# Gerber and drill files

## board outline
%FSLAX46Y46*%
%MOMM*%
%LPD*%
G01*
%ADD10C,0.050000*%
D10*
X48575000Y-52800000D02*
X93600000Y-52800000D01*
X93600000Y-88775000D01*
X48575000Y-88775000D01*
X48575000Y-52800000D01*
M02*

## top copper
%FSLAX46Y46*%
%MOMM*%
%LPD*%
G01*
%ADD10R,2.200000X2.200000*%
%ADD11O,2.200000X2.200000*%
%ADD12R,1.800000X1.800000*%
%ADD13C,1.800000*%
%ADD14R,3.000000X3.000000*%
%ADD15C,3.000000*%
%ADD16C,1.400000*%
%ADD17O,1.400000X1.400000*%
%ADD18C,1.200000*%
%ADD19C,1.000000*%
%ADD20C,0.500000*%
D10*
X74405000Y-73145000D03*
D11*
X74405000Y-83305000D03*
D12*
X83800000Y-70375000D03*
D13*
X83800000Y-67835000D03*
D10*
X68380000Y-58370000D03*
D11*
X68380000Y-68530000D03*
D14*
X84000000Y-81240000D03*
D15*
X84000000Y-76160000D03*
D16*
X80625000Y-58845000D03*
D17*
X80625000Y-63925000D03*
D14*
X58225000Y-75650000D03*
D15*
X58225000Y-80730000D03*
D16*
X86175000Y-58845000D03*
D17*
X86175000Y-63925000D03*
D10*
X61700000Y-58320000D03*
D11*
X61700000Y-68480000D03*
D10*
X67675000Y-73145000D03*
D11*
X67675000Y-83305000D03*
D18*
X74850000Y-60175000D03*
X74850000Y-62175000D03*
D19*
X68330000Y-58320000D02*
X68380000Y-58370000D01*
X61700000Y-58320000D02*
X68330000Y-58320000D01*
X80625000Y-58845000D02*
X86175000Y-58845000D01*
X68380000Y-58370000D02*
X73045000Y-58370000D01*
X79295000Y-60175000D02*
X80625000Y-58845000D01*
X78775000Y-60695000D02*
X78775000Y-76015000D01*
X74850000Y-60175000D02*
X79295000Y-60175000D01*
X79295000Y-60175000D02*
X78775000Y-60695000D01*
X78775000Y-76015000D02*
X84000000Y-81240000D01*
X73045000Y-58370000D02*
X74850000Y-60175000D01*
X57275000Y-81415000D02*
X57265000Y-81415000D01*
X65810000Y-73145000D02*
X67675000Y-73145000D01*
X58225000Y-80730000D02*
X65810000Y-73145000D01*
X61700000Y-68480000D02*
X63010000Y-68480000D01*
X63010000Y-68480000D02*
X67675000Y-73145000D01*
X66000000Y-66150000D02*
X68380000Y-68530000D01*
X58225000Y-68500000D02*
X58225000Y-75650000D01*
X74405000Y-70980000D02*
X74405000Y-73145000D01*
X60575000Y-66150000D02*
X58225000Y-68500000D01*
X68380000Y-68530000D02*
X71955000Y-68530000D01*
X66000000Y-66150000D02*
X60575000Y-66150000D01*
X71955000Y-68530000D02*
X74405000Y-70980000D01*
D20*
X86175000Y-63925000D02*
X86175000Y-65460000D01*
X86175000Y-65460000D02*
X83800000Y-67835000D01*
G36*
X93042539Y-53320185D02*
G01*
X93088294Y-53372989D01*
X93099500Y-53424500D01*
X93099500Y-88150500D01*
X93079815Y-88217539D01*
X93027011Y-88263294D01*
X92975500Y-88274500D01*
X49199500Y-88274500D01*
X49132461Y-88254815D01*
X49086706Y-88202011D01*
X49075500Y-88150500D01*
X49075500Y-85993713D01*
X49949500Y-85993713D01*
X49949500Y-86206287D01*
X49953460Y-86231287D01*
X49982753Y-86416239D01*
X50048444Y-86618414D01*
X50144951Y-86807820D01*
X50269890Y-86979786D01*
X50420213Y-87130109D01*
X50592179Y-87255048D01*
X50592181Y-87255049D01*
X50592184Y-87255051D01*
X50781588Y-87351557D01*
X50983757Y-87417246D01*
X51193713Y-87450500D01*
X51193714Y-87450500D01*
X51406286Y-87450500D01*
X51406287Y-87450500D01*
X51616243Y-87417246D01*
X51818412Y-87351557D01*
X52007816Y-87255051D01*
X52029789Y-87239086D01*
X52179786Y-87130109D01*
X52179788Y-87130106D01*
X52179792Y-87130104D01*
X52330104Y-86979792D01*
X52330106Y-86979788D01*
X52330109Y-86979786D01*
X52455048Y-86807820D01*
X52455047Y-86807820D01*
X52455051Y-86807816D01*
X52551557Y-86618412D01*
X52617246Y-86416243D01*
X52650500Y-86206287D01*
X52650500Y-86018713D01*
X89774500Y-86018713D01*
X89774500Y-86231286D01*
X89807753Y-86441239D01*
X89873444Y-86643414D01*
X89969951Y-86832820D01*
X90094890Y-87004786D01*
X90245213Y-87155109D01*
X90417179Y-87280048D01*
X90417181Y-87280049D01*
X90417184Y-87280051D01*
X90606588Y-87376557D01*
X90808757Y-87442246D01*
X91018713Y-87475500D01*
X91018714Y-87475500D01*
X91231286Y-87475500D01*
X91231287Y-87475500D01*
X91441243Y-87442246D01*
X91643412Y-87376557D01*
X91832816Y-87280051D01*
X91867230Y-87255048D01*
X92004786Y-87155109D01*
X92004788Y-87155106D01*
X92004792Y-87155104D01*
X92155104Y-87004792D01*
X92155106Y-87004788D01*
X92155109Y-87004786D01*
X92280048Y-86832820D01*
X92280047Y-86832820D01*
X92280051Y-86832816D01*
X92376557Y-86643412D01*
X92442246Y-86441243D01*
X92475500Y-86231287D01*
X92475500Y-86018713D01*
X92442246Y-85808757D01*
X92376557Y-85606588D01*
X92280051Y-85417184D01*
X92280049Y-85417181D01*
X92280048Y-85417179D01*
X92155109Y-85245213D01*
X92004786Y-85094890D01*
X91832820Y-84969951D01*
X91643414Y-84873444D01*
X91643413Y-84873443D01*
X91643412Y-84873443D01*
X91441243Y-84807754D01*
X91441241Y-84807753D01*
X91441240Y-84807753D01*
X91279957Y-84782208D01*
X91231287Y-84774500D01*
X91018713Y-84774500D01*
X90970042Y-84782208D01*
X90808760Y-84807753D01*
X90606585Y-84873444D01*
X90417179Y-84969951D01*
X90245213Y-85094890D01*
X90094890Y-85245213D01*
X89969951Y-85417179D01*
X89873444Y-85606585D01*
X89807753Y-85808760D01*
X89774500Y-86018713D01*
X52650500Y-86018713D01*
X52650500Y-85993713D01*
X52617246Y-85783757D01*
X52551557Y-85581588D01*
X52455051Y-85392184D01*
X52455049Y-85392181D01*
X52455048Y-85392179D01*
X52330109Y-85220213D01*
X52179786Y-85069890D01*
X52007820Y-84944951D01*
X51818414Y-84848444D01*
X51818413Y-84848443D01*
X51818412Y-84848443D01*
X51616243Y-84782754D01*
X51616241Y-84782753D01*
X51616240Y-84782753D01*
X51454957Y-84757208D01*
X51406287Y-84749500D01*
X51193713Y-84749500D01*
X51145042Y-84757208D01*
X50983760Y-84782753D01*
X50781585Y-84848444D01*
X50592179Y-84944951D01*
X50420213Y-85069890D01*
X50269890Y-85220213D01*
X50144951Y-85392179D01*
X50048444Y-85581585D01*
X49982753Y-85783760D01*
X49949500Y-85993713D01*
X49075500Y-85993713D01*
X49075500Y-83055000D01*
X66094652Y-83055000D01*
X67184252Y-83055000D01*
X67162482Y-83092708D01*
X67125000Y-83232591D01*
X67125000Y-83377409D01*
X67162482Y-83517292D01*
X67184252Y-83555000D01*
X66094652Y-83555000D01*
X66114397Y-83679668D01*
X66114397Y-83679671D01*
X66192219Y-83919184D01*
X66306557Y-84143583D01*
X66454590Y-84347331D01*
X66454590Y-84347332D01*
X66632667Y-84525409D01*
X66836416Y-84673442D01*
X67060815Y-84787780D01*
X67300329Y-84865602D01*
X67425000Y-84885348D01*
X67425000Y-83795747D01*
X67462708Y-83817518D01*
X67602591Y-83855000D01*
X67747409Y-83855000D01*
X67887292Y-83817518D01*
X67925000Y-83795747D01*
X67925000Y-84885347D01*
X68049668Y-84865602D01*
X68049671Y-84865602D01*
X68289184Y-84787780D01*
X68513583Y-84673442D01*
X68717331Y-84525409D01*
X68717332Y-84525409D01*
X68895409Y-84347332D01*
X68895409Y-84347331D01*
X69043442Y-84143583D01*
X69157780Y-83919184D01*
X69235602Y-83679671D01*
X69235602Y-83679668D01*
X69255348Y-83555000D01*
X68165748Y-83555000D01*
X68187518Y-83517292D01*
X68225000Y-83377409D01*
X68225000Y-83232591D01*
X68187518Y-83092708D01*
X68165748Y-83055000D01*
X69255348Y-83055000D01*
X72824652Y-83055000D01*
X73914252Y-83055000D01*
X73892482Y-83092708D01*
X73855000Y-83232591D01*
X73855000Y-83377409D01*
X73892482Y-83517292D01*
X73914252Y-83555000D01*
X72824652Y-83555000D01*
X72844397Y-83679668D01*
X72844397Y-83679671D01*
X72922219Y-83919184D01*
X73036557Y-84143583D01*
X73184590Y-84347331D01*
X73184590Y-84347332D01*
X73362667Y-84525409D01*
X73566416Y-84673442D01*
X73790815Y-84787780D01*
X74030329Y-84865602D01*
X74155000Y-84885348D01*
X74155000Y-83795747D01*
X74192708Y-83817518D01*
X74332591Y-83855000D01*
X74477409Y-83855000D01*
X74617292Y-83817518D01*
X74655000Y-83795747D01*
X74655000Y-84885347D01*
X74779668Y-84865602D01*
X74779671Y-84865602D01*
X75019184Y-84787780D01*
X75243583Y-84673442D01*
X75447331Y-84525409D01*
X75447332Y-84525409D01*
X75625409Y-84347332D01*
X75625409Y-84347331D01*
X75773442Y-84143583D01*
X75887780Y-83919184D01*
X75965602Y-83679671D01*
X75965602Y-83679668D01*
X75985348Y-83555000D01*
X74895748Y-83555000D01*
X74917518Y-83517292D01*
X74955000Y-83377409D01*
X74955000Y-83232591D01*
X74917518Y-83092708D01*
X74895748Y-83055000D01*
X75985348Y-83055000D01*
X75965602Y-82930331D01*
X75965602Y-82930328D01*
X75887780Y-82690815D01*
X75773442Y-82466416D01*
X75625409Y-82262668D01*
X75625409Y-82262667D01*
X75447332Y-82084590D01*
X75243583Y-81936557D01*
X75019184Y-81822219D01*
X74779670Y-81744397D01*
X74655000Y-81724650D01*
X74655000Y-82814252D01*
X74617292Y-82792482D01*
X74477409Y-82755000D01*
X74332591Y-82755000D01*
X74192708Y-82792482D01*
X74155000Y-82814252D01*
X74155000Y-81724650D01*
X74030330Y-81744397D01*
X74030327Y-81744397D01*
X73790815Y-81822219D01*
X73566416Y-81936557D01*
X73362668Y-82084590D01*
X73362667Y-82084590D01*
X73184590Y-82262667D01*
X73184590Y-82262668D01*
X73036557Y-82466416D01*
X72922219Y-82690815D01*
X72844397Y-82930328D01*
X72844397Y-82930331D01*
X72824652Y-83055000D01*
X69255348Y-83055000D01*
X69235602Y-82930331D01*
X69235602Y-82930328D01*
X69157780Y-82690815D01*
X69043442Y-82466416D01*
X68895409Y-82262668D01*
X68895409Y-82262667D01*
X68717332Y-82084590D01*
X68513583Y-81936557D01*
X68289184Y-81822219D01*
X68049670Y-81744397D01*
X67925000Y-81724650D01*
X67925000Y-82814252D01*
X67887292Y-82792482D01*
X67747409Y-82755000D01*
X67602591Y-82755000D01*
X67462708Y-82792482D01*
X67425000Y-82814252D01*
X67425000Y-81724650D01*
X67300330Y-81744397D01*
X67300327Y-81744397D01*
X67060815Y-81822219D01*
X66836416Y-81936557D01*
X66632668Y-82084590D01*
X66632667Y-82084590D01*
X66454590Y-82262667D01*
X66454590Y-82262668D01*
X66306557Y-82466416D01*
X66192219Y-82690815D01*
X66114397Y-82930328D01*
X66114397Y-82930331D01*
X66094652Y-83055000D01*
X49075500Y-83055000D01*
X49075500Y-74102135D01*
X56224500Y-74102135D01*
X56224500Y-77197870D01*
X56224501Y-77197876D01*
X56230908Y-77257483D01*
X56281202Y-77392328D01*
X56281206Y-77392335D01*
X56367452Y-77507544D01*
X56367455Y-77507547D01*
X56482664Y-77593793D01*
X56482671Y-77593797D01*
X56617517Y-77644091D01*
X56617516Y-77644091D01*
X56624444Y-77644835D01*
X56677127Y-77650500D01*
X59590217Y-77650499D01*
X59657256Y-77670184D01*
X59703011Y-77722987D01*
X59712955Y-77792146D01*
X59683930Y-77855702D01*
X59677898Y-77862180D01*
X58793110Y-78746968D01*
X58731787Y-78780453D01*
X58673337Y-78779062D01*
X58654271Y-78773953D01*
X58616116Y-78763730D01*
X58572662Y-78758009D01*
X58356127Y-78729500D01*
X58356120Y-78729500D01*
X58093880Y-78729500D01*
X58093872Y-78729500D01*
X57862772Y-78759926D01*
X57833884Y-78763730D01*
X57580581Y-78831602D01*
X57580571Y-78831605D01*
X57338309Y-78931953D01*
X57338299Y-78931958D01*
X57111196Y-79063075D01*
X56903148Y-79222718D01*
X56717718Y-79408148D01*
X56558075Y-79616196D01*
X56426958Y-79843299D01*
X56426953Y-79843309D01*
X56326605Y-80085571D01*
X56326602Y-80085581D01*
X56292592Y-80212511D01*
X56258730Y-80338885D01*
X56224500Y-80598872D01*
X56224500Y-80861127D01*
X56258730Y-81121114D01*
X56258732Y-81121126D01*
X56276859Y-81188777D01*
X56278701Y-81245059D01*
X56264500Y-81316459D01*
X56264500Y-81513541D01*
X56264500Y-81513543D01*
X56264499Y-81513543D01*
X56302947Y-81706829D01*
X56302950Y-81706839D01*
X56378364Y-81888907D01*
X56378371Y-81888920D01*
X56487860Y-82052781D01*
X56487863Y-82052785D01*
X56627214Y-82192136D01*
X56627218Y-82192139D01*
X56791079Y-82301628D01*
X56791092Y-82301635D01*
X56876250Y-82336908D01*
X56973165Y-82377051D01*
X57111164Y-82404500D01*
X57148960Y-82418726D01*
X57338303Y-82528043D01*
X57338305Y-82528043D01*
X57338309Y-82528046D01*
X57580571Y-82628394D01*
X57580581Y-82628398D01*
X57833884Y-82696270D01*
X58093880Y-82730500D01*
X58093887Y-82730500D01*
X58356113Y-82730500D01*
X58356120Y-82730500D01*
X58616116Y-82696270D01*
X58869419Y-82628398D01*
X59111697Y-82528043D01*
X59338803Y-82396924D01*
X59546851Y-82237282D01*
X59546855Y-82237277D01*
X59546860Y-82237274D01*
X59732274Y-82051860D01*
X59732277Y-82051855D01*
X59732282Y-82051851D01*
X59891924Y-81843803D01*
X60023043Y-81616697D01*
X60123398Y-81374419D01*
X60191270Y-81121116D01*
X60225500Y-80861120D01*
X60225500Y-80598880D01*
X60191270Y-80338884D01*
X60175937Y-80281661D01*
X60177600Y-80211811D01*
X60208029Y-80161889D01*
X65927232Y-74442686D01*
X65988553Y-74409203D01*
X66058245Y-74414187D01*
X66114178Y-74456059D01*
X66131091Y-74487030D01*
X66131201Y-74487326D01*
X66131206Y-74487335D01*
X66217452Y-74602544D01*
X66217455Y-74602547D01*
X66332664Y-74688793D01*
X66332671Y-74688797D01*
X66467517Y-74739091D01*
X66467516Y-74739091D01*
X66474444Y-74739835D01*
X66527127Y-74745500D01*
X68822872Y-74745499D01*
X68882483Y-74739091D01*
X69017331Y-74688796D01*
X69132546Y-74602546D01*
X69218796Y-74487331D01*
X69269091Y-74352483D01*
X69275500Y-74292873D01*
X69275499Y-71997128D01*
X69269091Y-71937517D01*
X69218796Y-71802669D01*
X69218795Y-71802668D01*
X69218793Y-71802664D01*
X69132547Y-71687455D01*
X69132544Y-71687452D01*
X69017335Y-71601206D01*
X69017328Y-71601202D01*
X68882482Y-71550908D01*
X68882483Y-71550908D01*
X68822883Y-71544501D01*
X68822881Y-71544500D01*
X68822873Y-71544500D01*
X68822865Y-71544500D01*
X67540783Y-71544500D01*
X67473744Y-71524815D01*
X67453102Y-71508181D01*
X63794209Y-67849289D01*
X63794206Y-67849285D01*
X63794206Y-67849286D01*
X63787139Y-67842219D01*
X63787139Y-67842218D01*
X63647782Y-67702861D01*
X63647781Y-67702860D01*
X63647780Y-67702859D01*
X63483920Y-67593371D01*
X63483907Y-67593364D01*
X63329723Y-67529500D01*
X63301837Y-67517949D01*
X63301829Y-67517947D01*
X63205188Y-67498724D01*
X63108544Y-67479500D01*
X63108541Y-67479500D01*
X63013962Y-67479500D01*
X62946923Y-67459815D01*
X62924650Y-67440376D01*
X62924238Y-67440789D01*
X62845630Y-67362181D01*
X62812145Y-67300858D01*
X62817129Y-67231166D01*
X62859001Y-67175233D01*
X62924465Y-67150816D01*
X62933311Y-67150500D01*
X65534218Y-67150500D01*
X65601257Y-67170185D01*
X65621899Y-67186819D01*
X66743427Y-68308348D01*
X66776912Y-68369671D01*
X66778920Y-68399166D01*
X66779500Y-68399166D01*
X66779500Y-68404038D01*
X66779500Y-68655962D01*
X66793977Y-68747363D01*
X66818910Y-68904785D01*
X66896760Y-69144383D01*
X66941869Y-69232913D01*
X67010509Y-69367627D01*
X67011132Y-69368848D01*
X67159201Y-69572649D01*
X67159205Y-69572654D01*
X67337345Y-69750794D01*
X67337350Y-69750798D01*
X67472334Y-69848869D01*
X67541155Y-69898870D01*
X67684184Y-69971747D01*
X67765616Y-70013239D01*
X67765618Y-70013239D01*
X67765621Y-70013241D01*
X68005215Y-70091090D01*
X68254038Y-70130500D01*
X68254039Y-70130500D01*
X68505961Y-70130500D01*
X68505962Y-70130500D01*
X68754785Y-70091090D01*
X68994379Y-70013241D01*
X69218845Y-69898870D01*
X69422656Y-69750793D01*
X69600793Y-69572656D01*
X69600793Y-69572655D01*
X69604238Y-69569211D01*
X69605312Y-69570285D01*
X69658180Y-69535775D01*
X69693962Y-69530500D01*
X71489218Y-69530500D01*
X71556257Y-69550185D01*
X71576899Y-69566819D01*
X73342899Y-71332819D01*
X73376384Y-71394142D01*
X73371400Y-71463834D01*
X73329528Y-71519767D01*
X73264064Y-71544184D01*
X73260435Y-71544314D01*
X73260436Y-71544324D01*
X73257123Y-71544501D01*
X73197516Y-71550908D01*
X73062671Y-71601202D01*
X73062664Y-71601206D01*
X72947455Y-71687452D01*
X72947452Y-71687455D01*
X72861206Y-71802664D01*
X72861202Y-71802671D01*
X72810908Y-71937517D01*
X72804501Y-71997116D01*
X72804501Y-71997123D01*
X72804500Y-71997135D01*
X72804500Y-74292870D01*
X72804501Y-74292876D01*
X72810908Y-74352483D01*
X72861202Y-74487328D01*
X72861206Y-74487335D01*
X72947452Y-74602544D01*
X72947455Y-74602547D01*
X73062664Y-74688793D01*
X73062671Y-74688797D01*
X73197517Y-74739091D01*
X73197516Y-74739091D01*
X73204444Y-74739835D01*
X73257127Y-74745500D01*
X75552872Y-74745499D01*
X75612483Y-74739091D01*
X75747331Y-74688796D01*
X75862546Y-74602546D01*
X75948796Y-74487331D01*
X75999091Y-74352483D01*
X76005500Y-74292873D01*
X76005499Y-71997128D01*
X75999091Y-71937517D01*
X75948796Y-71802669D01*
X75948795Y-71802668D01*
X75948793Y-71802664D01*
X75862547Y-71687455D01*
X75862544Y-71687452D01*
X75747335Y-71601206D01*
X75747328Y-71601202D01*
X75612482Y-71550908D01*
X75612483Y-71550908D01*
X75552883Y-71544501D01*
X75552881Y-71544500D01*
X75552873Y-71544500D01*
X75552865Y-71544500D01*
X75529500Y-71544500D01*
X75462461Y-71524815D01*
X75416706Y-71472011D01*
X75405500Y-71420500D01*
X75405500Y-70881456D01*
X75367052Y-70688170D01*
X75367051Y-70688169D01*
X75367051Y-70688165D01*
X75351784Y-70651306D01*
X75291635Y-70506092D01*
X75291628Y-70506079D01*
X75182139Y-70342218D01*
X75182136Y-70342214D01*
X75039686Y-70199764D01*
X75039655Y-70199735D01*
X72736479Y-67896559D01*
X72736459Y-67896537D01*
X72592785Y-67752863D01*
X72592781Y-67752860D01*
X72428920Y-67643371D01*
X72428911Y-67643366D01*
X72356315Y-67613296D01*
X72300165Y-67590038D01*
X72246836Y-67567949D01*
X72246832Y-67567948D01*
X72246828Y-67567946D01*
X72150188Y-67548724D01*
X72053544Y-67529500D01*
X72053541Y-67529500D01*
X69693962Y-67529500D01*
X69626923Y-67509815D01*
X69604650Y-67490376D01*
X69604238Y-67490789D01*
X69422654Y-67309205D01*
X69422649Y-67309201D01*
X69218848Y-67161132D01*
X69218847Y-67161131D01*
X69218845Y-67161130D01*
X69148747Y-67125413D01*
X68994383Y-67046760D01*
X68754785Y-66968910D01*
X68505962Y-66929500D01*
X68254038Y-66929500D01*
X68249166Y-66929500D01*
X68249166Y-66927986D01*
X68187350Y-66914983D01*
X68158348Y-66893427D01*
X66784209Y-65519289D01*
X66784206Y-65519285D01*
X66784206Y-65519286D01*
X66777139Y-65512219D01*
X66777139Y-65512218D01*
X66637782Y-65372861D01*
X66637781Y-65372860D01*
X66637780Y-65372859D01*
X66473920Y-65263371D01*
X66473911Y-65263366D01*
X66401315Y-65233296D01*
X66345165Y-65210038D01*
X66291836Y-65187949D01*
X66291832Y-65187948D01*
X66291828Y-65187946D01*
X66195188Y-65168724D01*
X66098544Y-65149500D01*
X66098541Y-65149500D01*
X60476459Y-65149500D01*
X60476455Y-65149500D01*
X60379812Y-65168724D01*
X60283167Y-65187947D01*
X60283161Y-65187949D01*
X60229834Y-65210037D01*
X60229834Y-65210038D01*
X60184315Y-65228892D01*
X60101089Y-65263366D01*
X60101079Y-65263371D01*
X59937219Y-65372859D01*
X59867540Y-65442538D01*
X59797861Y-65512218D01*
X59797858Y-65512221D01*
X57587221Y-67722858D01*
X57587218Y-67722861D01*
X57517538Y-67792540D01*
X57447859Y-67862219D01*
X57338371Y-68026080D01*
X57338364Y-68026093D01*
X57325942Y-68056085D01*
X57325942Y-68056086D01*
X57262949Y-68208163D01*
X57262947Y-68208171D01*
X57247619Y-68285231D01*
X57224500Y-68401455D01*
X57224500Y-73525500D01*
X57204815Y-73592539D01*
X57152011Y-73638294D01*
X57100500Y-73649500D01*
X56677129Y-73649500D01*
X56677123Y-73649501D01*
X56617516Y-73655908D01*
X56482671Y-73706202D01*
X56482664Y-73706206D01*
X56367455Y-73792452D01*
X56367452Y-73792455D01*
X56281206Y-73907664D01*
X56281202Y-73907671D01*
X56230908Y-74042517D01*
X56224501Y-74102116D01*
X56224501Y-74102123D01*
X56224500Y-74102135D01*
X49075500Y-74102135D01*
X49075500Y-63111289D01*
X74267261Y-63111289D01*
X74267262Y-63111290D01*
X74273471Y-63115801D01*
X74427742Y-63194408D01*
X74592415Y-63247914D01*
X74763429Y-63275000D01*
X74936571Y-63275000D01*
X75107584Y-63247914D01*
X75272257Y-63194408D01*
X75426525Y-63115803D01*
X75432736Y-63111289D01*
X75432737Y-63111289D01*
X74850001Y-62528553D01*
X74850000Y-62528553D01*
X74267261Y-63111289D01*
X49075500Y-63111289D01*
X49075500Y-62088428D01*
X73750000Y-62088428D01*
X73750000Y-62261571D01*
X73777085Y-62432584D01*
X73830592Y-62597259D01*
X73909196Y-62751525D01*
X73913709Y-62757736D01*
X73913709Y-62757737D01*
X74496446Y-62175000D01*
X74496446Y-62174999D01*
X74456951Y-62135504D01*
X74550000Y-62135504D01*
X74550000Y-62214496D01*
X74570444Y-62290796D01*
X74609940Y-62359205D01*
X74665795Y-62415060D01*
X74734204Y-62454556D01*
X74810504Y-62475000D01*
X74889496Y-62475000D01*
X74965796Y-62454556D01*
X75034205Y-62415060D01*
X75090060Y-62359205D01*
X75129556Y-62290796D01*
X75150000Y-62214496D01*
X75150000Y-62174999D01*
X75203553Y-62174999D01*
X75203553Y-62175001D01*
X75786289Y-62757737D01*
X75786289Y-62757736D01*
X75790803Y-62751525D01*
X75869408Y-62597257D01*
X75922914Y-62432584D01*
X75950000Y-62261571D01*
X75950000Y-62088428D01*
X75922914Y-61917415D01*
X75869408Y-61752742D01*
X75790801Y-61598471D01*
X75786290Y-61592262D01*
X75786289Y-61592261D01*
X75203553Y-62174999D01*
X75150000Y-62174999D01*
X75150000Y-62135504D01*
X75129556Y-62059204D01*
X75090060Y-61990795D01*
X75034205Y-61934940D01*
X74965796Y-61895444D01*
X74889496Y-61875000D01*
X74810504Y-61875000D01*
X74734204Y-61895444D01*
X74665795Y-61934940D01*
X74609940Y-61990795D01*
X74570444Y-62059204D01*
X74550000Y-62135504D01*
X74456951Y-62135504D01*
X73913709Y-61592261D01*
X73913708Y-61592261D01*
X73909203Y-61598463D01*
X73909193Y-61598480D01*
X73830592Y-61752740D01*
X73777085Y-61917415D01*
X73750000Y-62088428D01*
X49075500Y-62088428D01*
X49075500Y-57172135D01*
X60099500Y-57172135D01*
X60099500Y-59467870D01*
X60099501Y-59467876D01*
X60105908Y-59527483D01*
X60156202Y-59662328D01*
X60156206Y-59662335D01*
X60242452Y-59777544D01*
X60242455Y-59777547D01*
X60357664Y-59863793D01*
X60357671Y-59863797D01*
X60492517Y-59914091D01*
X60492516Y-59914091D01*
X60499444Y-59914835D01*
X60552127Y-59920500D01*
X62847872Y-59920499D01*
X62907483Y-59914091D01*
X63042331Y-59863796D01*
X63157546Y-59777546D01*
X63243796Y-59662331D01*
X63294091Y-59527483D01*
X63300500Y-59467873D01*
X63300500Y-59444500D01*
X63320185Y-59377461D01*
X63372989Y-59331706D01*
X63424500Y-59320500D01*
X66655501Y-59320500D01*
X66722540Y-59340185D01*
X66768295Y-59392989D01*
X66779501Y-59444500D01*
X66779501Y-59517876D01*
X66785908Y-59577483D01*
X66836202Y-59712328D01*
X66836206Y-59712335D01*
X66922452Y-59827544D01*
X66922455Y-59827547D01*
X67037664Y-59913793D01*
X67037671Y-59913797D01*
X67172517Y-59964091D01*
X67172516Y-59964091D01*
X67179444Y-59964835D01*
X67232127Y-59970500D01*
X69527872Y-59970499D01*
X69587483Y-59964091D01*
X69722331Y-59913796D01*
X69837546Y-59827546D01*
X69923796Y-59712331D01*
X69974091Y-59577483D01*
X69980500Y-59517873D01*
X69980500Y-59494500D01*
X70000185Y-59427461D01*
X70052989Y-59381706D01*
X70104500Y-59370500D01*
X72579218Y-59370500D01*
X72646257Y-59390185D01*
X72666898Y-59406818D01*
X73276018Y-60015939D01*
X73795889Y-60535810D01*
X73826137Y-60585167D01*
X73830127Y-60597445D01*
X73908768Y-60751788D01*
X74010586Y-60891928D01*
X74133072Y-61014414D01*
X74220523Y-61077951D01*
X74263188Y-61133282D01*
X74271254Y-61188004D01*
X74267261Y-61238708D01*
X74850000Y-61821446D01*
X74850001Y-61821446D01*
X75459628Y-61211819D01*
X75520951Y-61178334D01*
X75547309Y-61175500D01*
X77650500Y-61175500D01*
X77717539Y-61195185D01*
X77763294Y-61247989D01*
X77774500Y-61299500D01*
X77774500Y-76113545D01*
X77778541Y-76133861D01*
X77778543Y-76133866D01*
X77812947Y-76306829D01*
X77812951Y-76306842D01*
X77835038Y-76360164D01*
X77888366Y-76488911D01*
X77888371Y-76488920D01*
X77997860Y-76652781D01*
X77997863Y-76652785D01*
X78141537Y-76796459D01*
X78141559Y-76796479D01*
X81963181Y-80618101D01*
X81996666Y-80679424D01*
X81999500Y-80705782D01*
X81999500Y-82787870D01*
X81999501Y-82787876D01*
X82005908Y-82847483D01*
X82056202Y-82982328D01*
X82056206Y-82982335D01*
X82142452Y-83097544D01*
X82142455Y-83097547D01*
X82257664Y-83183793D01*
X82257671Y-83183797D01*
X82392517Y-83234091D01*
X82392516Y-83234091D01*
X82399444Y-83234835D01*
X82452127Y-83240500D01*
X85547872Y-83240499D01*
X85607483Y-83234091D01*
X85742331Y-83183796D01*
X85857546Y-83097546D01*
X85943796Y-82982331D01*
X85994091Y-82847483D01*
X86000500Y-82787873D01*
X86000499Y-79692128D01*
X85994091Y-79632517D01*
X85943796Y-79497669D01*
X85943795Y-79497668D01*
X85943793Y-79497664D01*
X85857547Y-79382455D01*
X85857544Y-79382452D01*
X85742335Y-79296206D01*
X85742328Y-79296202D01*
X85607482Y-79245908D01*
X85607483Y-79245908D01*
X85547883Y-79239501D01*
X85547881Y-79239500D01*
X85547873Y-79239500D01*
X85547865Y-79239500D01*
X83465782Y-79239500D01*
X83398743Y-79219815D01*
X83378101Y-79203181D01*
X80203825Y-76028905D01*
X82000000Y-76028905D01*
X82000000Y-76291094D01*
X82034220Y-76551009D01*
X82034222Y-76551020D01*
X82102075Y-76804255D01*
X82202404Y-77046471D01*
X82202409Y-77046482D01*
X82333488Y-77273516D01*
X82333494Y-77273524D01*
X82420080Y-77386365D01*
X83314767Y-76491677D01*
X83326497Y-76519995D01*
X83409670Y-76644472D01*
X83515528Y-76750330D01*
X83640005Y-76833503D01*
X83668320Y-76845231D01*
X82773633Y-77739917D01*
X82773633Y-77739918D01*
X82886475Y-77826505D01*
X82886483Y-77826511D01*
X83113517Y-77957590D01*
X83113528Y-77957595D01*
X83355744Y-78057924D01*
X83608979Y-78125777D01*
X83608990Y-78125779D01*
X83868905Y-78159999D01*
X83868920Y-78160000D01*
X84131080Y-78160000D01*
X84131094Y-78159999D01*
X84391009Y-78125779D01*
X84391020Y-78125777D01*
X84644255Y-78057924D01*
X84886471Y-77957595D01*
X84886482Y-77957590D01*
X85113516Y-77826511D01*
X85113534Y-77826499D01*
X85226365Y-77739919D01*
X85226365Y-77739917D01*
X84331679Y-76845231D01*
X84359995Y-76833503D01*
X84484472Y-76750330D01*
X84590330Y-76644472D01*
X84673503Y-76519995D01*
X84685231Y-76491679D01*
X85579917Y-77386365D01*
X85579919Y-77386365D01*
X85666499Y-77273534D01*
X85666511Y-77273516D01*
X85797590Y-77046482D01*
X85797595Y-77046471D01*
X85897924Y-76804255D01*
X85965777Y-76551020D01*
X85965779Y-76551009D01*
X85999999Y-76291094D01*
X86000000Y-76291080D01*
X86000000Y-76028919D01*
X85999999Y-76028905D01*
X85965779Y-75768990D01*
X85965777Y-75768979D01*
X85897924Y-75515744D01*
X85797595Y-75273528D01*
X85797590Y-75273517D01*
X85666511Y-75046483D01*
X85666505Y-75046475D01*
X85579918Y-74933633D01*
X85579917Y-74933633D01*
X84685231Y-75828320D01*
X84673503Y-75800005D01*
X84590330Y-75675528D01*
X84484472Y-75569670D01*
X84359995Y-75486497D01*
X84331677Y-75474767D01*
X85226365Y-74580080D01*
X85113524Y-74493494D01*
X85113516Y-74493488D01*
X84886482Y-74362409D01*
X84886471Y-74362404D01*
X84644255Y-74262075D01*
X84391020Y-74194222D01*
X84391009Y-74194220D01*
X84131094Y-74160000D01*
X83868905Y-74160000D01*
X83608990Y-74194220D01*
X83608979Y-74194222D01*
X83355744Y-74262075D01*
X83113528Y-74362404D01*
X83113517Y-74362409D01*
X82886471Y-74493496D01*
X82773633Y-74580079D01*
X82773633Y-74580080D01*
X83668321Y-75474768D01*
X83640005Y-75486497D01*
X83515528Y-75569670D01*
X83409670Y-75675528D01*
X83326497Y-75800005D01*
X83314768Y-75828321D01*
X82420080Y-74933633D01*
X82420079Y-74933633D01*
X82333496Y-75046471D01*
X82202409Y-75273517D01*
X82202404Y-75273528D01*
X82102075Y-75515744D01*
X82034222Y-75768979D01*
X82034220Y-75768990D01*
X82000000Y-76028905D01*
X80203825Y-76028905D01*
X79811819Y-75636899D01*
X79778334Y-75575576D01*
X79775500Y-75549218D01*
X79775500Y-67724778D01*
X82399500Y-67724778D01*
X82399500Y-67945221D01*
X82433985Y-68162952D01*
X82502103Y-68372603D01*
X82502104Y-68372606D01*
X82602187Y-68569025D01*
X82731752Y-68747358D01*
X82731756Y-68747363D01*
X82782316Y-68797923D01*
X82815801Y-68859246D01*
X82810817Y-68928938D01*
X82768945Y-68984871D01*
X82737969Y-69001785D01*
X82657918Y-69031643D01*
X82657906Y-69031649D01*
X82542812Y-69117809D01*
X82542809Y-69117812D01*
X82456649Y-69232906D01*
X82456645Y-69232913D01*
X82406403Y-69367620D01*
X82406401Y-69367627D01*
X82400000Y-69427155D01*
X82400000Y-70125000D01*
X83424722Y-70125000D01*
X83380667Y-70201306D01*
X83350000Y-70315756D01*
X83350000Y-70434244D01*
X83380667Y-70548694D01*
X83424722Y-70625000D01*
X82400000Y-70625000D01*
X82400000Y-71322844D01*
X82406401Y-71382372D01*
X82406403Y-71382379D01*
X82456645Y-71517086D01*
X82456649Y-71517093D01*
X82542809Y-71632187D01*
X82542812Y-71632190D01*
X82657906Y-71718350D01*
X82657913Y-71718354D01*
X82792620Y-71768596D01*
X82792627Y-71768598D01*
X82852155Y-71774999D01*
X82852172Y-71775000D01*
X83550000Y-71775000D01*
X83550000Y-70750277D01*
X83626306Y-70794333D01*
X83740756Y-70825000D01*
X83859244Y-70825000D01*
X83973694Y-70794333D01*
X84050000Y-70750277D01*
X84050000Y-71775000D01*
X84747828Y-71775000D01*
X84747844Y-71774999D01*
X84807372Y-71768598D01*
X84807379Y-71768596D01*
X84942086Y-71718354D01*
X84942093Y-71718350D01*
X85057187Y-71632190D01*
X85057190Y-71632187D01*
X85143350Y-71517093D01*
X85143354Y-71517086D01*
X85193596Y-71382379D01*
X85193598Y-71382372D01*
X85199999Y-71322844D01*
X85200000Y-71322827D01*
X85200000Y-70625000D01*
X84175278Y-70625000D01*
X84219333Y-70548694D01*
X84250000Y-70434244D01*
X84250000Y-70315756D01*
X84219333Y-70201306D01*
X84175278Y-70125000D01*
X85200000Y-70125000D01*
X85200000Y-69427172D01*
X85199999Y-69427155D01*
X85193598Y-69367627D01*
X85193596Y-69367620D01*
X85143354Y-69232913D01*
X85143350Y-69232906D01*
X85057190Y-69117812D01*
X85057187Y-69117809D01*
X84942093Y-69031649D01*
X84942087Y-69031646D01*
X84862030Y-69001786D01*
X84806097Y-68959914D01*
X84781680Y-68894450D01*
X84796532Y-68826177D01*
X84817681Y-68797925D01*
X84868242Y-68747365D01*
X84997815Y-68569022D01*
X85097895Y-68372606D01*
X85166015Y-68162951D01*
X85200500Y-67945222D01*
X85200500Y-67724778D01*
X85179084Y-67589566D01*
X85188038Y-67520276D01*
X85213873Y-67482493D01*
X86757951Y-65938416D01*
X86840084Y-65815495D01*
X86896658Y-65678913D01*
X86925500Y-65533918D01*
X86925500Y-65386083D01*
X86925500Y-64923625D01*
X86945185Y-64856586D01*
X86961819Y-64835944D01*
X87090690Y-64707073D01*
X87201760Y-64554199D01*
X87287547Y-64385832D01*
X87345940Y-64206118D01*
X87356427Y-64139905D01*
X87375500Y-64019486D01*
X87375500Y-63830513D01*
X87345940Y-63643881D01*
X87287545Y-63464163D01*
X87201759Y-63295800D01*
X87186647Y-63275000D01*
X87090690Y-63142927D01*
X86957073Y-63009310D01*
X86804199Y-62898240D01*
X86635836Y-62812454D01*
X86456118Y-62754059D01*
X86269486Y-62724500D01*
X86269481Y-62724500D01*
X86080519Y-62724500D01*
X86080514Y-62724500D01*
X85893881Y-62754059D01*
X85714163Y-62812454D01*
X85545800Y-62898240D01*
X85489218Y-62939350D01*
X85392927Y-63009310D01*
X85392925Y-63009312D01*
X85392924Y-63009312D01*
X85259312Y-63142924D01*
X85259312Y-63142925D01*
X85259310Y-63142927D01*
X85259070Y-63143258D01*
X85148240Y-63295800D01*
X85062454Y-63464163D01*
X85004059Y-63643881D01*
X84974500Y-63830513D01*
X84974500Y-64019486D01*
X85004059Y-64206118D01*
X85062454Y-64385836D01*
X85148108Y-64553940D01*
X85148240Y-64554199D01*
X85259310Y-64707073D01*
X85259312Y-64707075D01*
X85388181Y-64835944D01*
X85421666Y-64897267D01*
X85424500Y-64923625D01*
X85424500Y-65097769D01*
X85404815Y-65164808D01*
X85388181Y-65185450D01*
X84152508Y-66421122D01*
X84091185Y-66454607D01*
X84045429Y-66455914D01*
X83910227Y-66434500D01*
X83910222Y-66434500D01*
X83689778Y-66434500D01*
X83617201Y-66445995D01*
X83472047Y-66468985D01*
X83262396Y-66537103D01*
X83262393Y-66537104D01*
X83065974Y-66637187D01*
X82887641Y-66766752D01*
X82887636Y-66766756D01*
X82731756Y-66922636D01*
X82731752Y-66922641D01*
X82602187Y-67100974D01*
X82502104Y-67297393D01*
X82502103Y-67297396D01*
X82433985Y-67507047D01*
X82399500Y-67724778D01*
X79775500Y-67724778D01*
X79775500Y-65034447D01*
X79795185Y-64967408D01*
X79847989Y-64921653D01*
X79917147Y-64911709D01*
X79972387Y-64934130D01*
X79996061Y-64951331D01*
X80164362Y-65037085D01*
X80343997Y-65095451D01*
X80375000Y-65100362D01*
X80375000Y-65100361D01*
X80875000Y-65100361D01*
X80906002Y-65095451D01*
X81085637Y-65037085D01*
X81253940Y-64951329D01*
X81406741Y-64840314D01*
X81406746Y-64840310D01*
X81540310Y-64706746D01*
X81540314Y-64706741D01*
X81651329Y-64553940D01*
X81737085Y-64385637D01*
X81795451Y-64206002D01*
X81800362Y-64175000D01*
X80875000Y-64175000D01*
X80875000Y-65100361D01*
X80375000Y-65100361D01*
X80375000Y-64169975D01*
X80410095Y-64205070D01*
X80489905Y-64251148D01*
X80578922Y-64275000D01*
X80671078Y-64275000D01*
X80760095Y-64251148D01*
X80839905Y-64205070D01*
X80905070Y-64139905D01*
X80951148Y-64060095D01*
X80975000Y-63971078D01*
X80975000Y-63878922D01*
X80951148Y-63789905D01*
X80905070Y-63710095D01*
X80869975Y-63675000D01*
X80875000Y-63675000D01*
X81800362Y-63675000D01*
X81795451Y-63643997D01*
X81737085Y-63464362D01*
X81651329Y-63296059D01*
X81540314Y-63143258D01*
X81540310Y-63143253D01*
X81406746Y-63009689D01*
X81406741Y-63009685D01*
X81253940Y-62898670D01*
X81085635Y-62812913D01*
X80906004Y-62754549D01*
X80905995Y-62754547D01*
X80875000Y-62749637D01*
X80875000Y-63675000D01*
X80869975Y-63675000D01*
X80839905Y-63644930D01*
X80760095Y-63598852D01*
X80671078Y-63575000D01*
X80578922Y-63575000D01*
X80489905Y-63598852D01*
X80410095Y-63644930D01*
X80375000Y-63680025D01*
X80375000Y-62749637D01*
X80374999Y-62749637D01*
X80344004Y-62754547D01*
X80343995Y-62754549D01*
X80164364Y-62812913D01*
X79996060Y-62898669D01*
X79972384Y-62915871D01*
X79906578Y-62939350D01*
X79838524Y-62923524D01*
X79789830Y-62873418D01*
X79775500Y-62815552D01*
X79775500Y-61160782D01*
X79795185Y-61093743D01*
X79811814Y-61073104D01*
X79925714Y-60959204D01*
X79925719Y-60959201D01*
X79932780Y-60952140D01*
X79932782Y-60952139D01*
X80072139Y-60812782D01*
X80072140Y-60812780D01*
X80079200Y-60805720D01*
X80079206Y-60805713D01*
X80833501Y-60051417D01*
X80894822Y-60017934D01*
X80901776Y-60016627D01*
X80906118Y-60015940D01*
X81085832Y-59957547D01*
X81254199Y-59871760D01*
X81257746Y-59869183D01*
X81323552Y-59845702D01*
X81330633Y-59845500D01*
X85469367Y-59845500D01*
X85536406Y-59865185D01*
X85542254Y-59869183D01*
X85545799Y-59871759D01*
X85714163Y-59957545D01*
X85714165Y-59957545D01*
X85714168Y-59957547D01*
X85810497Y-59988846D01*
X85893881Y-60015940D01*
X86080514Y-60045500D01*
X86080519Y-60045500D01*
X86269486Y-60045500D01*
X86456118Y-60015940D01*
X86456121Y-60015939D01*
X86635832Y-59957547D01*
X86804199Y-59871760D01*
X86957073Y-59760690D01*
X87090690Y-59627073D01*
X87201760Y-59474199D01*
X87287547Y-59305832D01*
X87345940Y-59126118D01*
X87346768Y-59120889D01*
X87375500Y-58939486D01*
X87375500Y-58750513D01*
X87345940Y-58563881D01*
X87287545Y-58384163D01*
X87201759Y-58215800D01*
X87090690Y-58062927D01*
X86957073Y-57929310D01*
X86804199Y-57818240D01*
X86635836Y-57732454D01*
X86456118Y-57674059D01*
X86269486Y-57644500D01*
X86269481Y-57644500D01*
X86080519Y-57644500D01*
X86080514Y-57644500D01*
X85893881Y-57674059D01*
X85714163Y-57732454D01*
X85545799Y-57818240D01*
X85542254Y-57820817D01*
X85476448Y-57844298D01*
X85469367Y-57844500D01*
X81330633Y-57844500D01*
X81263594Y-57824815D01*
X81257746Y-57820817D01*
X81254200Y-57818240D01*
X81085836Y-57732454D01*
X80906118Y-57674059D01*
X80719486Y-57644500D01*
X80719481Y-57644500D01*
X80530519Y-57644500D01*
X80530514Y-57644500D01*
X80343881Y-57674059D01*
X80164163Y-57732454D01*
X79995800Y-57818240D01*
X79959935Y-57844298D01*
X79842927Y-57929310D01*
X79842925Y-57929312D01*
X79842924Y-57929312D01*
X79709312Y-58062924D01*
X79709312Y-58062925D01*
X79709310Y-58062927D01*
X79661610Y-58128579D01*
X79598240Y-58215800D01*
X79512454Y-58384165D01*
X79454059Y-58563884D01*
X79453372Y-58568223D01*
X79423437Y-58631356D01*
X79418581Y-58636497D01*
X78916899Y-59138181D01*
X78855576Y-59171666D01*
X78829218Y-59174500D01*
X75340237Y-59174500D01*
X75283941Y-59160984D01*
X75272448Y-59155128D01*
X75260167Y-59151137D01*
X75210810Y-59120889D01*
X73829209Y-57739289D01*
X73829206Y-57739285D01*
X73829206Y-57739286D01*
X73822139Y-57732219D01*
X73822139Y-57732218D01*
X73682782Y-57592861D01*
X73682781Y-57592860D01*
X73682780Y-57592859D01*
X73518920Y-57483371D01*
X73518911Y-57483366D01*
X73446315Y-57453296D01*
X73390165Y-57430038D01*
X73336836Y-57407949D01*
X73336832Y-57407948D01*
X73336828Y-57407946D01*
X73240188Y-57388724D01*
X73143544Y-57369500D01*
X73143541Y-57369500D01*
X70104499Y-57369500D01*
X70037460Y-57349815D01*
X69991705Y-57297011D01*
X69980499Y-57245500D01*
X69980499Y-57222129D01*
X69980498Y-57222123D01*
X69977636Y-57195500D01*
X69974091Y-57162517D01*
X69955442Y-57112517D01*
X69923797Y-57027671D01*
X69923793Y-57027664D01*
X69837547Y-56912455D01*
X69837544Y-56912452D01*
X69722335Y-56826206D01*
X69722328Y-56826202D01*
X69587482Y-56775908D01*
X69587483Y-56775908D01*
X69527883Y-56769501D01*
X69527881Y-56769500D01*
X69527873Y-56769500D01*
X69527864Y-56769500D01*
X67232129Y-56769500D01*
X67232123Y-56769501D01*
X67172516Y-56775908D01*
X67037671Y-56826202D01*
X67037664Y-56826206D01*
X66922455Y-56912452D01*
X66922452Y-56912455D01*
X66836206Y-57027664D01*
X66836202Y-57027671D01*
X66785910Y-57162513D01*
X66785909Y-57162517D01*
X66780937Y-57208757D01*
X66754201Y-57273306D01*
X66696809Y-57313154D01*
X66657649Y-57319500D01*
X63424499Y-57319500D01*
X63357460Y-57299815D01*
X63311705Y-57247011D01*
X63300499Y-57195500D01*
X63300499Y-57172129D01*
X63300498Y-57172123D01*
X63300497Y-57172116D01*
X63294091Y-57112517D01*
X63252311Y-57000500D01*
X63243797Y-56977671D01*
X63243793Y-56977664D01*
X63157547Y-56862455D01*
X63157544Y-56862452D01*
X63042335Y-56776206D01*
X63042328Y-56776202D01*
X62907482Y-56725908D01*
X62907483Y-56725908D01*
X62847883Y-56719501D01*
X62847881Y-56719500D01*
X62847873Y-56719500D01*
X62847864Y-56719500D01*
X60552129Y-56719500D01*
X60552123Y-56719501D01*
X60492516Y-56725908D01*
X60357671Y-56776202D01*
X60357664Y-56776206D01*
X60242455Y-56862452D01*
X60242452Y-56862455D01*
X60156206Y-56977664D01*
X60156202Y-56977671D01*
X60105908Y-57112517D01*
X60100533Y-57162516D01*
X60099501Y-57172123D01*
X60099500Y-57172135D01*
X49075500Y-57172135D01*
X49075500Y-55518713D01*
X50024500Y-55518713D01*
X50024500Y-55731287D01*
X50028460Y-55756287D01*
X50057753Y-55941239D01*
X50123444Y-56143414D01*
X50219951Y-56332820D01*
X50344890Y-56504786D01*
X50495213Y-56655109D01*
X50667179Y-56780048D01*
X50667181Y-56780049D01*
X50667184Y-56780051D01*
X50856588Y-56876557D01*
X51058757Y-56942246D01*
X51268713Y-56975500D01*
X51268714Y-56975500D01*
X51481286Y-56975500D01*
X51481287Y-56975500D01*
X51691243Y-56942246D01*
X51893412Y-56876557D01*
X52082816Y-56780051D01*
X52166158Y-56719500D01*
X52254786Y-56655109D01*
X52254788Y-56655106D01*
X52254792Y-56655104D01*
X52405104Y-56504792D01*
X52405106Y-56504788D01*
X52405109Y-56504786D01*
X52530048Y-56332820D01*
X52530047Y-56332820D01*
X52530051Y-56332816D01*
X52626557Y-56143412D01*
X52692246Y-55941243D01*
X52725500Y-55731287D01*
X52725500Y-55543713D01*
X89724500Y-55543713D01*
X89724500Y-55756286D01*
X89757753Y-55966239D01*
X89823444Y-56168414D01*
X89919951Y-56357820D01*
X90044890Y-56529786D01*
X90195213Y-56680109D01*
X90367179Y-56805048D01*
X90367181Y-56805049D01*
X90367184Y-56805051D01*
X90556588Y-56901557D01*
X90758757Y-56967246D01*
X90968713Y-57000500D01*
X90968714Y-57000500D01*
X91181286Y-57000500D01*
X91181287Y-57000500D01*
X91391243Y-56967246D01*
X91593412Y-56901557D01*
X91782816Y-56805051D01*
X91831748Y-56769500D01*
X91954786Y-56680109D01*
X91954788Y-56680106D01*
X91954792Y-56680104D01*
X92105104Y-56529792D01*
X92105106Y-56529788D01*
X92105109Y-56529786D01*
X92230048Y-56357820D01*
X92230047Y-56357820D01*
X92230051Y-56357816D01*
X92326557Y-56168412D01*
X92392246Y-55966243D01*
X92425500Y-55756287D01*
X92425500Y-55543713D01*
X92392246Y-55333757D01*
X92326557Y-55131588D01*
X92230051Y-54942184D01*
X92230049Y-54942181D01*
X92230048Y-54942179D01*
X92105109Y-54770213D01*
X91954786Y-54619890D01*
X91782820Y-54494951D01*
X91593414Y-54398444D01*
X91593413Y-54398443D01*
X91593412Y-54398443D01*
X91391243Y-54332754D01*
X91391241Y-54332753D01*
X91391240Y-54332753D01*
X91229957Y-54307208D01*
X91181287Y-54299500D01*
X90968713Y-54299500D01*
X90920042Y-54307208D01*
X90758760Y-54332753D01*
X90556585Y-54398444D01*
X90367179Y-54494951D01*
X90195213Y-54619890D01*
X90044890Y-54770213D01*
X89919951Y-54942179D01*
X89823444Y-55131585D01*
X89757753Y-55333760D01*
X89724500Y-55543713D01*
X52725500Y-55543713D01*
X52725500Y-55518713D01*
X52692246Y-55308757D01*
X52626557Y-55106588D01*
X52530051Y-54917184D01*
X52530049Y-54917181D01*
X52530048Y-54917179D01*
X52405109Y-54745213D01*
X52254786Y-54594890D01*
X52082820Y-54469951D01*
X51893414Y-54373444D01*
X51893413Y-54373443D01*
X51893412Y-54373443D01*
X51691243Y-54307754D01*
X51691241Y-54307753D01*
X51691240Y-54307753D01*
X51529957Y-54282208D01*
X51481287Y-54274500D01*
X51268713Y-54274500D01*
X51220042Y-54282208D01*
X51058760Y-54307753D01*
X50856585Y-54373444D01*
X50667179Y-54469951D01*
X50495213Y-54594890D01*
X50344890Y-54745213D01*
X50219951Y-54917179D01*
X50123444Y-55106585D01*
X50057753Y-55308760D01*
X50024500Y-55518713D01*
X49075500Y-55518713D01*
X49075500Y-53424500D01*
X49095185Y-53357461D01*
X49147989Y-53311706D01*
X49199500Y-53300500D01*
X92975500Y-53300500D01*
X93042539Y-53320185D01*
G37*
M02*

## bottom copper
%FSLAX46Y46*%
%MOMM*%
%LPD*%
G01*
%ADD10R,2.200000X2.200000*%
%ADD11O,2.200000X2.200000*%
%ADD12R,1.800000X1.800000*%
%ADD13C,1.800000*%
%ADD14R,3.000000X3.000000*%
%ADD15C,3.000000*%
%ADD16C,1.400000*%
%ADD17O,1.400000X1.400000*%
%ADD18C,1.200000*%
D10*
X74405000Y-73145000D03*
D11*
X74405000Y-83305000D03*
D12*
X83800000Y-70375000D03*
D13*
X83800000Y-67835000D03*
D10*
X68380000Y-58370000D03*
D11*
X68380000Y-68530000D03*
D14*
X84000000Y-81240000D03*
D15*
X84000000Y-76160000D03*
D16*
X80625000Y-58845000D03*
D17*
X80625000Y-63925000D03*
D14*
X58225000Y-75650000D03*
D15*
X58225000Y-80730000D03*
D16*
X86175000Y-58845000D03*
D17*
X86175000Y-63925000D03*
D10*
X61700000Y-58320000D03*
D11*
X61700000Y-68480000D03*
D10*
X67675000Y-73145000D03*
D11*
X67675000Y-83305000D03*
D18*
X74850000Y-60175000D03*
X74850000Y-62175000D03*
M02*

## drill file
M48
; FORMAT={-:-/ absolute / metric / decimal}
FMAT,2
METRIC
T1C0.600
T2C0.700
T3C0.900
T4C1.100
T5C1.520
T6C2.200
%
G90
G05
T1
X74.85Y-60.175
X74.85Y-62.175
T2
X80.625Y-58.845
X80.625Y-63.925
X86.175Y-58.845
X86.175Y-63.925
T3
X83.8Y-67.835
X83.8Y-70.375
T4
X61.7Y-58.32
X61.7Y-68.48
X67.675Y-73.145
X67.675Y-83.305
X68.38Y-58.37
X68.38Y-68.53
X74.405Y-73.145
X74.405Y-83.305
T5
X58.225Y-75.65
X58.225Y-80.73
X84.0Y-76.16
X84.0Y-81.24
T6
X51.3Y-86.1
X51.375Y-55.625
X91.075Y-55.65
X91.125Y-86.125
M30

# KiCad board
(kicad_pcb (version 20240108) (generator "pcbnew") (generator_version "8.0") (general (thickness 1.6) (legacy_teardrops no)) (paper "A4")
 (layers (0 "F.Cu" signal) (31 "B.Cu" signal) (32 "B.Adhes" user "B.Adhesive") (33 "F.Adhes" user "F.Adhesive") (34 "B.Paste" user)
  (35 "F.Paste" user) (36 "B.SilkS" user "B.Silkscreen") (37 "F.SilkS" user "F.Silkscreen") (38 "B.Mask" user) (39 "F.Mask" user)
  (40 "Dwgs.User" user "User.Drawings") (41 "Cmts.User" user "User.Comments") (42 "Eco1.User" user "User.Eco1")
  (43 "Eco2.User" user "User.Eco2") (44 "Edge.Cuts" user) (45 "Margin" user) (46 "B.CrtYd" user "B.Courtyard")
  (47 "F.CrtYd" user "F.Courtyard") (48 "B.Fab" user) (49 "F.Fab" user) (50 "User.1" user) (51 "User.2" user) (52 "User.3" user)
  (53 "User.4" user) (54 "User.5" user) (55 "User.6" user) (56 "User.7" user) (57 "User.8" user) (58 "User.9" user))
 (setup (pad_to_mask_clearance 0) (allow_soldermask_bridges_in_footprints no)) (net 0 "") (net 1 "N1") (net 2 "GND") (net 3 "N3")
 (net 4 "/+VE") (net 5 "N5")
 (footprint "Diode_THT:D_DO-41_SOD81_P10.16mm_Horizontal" (layer "F.Cu") (at 74.405 73.145 -90)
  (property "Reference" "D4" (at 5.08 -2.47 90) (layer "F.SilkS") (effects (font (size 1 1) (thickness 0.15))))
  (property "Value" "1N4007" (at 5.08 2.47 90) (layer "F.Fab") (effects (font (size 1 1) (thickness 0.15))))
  (pad "1" thru_hole rect (at 0 0 270) (size 2.2 2.2) (drill 1.1) (layers "*.Cu" "*.Mask") (remove_unused_layers no) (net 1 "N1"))
  (pad "2" thru_hole oval (at 10.16 0 270) (size 2.2 2.2) (drill 1.1) (layers "*.Cu" "*.Mask") (remove_unused_layers no) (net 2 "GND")))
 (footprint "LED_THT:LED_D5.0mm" (layer "F.Cu") (at 83.8 70.375 90)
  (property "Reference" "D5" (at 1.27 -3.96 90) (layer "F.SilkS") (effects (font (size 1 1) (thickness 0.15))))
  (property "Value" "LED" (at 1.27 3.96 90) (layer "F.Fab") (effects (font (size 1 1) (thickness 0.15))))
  (pad "1" thru_hole rect (at 0 0 90) (size 1.8 1.8) (drill 0.9) (layers "*.Cu" "*.Mask") (remove_unused_layers no) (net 2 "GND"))
  (pad "2" thru_hole circle (at 2.54 0 90) (size 1.8 1.8) (drill 0.9) (layers "*.Cu" "*.Mask") (remove_unused_layers no) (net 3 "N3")))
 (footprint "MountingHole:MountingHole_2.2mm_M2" (layer "F.Cu") (at 51.375 55.625)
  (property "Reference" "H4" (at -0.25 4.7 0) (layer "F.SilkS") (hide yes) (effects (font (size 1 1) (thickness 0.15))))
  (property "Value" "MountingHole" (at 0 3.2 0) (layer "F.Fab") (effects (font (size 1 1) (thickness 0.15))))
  (pad "" np_thru_hole circle (at 0 0) (size 2.2 2.2) (drill 2.2) (layers "*.Cu" "*.Mask")))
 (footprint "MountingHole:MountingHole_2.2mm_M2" (layer "F.Cu") (at 91.125 86.125)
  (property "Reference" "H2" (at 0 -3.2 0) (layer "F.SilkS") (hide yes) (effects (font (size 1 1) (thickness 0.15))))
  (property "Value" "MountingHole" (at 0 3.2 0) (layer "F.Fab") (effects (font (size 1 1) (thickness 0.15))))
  (pad "" np_thru_hole circle (at 0 0) (size 2.2 2.2) (drill 2.2) (layers "*.Cu" "*.Mask")))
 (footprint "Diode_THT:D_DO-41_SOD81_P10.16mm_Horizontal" (layer "F.Cu") (at 68.38 58.37 -90)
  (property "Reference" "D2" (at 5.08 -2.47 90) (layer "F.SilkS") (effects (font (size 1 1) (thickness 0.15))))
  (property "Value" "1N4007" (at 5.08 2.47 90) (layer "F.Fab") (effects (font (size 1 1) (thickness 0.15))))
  (pad "1" thru_hole rect (at 0 0 270) (size 2.2 2.2) (drill 1.1) (layers "*.Cu" "*.Mask") (remove_unused_layers no) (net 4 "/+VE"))
  (pad "2" thru_hole oval (at 10.16 0 270) (size 2.2 2.2) (drill 1.1) (layers "*.Cu" "*.Mask") (remove_unused_layers no) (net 1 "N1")))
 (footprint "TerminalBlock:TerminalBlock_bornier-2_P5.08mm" (layer "F.Cu") (at 84 81.24 90)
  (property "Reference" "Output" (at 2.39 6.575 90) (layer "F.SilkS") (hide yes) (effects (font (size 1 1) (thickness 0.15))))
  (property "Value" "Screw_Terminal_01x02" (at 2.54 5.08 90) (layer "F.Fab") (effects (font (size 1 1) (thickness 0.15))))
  (pad "1" thru_hole rect (at 0 0 90) (size 3 3) (drill 1.52) (layers "*.Cu" "*.Mask") (remove_unused_layers no) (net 4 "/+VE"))
  (pad "2" thru_hole circle (at 5.08 0 90) (size 3 3) (drill 1.52) (layers "*.Cu" "*.Mask") (remove_unused_layers no) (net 2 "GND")))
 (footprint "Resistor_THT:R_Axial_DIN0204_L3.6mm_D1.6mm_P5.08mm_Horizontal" (layer "F.Cu") (at 80.625 58.845 -90)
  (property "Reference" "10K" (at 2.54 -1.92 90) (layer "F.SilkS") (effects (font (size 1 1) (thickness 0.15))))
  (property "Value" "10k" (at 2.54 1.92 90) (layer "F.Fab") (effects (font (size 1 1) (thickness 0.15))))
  (pad "1" thru_hole circle (at 0 0 270) (size 1.4 1.4) (drill 0.7) (layers "*.Cu" "*.Mask") (remove_unused_layers no) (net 4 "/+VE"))
  (pad "2" thru_hole oval (at 5.08 0 270) (size 1.4 1.4) (drill 0.7) (layers "*.Cu" "*.Mask") (remove_unused_layers no) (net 2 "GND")))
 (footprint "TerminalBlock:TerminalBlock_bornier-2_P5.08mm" (layer "F.Cu") (at 58.225 75.65 -90)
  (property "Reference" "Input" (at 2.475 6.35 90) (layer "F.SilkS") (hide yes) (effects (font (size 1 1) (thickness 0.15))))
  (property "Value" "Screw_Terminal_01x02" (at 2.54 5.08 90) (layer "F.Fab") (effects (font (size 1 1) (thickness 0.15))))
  (pad "1" thru_hole rect (at 0 0 270) (size 3 3) (drill 1.52) (layers "*.Cu" "*.Mask") (remove_unused_layers no) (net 1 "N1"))
  (pad "2" thru_hole circle (at 5.08 0 270) (size 3 3) (drill 1.52) (layers "*.Cu" "*.Mask") (remove_unused_layers no) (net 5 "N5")))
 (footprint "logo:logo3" (layer "F.Cu") (at 54.3 62.625)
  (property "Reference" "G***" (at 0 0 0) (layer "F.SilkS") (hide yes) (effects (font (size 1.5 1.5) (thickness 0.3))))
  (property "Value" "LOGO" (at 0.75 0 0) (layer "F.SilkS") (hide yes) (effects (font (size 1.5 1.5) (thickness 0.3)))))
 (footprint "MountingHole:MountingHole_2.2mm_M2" (layer "F.Cu") (at 51.3 86.1)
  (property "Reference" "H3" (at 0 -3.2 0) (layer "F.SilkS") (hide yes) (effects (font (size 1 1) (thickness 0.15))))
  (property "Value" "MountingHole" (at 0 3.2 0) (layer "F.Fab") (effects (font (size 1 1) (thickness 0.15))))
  (pad "" np_thru_hole circle (at 0 0) (size 2.2 2.2) (drill 2.2) (layers "*.Cu" "*.Mask")))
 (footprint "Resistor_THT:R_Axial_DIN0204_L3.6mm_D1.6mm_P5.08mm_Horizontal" (layer "F.Cu") (at 86.175 58.845 -90)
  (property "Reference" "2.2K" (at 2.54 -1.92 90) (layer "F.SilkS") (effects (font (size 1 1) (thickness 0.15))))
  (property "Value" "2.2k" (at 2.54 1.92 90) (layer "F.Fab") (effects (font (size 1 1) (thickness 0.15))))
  (pad "1" thru_hole circle (at 0 0 270) (size 1.4 1.4) (drill 0.7) (layers "*.Cu" "*.Mask") (remove_unused_layers no) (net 4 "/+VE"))
  (pad "2" thru_hole oval (at 5.08 0 270) (size 1.4 1.4) (drill 0.7) (layers "*.Cu" "*.Mask") (remove_unused_layers no) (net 3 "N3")))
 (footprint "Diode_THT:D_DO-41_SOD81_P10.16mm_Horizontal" (layer "F.Cu") (at 61.7 58.32 -90)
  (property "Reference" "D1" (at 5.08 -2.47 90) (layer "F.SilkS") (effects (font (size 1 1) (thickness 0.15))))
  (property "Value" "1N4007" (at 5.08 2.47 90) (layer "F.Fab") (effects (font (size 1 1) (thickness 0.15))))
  (pad "1" thru_hole rect (at 0 0 270) (size 2.2 2.2) (drill 1.1) (layers "*.Cu" "*.Mask") (remove_unused_layers no) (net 4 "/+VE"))
  (pad "2" thru_hole oval (at 10.16 0 270) (size 2.2 2.2) (drill 1.1) (layers "*.Cu" "*.Mask") (remove_unused_layers no) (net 5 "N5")))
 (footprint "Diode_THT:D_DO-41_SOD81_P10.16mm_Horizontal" (layer "F.Cu") (at 67.675 73.145 -90)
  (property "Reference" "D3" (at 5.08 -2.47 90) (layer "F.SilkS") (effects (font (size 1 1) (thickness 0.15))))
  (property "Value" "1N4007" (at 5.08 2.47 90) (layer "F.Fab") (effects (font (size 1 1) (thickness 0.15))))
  (pad "1" thru_hole rect (at 0 0 270) (size 2.2 2.2) (drill 1.1) (layers "*.Cu" "*.Mask") (remove_unused_layers no) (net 5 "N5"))
  (pad "2" thru_hole oval (at 10.16 0 270) (size 2.2 2.2) (drill 1.1) (layers "*.Cu" "*.Mask") (remove_unused_layers no) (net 2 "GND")))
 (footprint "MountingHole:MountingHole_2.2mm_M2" (layer "F.Cu") (at 91.075 55.65)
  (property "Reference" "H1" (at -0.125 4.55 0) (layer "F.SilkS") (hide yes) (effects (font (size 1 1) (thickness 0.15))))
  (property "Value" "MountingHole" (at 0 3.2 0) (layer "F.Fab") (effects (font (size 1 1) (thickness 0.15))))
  (pad "" np_thru_hole circle (at 0 0) (size 2.2 2.2) (drill 2.2) (layers "*.Cu" "*.Mask")))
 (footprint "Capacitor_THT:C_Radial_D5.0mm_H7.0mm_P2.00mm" (layer "F.Cu") (at 74.85 60.175 -90)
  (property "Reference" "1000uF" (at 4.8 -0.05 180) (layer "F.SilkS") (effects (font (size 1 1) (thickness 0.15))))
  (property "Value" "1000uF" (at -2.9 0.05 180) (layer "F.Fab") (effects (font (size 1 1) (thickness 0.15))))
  (pad "1" thru_hole circle (at 0 0 270) (size 1.2 1.2) (drill 0.6) (layers "*.Cu" "*.Mask") (remove_unused_layers no) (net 4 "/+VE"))
  (pad "2" thru_hole circle (at 2 0 270) (size 1.2 1.2) (drill 0.6) (layers "*.Cu" "*.Mask") (remove_unused_layers no) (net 2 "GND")))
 (gr_rect (start 48.575 52.8) (end 93.6 88.775) (stroke (width 0.05) (type default)) (fill none) (layer "Edge.Cuts"))
 (segment (start 68.33 58.32) (end 68.38 58.37) (width 1) (layer "F.Cu") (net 4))
 (segment (start 61.7 58.32) (end 68.33 58.32) (width 1) (layer "F.Cu") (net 4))
 (segment (start 80.625 58.845) (end 86.175 58.845) (width 1) (layer "F.Cu") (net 4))
 (segment (start 68.38 58.37) (end 73.045 58.37) (width 1) (layer "F.Cu") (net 4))
 (segment (start 79.295 60.175) (end 80.625 58.845) (width 1) (layer "F.Cu") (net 4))
 (segment (start 78.775 60.695) (end 78.775 76.015) (width 1) (layer "F.Cu") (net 4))
 (segment (start 74.85 60.175) (end 79.295 60.175) (width 1) (layer "F.Cu") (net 4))
 (segment (start 79.295 60.175) (end 78.775 60.695) (width 1) (layer "F.Cu") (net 4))
 (segment (start 78.775 76.015) (end 84 81.24) (width 1) (layer "F.Cu") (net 4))
 (segment (start 73.045 58.37) (end 74.85 60.175) (width 1) (layer "F.Cu") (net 4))
 (segment (start 57.275 81.415) (end 57.265 81.415) (width 1) (layer "F.Cu") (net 5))
 (segment (start 65.81 73.145) (end 67.675 73.145) (width 1) (layer "F.Cu") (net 5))
 (segment (start 58.225 80.73) (end 65.81 73.145) (width 1) (layer "F.Cu") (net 5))
 (segment (start 61.7 68.48) (end 63.01 68.48) (width 1) (layer "F.Cu") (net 5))
 (segment (start 63.01 68.48) (end 67.675 73.145) (width 1) (layer "F.Cu") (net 5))
 (segment (start 66 66.15) (end 68.38 68.53) (width 1) (layer "F.Cu") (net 1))
 (segment (start 58.225 68.5) (end 58.225 75.65) (width 1) (layer "F.Cu") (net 1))
 (segment (start 74.405 70.98) (end 74.405 73.145) (width 1) (layer "F.Cu") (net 1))
 (segment (start 60.575 66.15) (end 58.225 68.5) (width 1) (layer "F.Cu") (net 1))
 (segment (start 68.38 68.53) (end 71.955 68.53) (width 1) (layer "F.Cu") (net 1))
 (segment (start 66 66.15) (end 60.575 66.15) (width 1) (layer "F.Cu") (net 1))
 (segment (start 71.955 68.53) (end 74.405 70.98) (width 1) (layer "F.Cu") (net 1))
 (segment (start 86.175 63.925) (end 86.175 65.46) (width 0.5) (layer "F.Cu") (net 3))
 (segment (start 86.175 65.46) (end 83.8 67.835) (width 0.5) (layer "F.Cu") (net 3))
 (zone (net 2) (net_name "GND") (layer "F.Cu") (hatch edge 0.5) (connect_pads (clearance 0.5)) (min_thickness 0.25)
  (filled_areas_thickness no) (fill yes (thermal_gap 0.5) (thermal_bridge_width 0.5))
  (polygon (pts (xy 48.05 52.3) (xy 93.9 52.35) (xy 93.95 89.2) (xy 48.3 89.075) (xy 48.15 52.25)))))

